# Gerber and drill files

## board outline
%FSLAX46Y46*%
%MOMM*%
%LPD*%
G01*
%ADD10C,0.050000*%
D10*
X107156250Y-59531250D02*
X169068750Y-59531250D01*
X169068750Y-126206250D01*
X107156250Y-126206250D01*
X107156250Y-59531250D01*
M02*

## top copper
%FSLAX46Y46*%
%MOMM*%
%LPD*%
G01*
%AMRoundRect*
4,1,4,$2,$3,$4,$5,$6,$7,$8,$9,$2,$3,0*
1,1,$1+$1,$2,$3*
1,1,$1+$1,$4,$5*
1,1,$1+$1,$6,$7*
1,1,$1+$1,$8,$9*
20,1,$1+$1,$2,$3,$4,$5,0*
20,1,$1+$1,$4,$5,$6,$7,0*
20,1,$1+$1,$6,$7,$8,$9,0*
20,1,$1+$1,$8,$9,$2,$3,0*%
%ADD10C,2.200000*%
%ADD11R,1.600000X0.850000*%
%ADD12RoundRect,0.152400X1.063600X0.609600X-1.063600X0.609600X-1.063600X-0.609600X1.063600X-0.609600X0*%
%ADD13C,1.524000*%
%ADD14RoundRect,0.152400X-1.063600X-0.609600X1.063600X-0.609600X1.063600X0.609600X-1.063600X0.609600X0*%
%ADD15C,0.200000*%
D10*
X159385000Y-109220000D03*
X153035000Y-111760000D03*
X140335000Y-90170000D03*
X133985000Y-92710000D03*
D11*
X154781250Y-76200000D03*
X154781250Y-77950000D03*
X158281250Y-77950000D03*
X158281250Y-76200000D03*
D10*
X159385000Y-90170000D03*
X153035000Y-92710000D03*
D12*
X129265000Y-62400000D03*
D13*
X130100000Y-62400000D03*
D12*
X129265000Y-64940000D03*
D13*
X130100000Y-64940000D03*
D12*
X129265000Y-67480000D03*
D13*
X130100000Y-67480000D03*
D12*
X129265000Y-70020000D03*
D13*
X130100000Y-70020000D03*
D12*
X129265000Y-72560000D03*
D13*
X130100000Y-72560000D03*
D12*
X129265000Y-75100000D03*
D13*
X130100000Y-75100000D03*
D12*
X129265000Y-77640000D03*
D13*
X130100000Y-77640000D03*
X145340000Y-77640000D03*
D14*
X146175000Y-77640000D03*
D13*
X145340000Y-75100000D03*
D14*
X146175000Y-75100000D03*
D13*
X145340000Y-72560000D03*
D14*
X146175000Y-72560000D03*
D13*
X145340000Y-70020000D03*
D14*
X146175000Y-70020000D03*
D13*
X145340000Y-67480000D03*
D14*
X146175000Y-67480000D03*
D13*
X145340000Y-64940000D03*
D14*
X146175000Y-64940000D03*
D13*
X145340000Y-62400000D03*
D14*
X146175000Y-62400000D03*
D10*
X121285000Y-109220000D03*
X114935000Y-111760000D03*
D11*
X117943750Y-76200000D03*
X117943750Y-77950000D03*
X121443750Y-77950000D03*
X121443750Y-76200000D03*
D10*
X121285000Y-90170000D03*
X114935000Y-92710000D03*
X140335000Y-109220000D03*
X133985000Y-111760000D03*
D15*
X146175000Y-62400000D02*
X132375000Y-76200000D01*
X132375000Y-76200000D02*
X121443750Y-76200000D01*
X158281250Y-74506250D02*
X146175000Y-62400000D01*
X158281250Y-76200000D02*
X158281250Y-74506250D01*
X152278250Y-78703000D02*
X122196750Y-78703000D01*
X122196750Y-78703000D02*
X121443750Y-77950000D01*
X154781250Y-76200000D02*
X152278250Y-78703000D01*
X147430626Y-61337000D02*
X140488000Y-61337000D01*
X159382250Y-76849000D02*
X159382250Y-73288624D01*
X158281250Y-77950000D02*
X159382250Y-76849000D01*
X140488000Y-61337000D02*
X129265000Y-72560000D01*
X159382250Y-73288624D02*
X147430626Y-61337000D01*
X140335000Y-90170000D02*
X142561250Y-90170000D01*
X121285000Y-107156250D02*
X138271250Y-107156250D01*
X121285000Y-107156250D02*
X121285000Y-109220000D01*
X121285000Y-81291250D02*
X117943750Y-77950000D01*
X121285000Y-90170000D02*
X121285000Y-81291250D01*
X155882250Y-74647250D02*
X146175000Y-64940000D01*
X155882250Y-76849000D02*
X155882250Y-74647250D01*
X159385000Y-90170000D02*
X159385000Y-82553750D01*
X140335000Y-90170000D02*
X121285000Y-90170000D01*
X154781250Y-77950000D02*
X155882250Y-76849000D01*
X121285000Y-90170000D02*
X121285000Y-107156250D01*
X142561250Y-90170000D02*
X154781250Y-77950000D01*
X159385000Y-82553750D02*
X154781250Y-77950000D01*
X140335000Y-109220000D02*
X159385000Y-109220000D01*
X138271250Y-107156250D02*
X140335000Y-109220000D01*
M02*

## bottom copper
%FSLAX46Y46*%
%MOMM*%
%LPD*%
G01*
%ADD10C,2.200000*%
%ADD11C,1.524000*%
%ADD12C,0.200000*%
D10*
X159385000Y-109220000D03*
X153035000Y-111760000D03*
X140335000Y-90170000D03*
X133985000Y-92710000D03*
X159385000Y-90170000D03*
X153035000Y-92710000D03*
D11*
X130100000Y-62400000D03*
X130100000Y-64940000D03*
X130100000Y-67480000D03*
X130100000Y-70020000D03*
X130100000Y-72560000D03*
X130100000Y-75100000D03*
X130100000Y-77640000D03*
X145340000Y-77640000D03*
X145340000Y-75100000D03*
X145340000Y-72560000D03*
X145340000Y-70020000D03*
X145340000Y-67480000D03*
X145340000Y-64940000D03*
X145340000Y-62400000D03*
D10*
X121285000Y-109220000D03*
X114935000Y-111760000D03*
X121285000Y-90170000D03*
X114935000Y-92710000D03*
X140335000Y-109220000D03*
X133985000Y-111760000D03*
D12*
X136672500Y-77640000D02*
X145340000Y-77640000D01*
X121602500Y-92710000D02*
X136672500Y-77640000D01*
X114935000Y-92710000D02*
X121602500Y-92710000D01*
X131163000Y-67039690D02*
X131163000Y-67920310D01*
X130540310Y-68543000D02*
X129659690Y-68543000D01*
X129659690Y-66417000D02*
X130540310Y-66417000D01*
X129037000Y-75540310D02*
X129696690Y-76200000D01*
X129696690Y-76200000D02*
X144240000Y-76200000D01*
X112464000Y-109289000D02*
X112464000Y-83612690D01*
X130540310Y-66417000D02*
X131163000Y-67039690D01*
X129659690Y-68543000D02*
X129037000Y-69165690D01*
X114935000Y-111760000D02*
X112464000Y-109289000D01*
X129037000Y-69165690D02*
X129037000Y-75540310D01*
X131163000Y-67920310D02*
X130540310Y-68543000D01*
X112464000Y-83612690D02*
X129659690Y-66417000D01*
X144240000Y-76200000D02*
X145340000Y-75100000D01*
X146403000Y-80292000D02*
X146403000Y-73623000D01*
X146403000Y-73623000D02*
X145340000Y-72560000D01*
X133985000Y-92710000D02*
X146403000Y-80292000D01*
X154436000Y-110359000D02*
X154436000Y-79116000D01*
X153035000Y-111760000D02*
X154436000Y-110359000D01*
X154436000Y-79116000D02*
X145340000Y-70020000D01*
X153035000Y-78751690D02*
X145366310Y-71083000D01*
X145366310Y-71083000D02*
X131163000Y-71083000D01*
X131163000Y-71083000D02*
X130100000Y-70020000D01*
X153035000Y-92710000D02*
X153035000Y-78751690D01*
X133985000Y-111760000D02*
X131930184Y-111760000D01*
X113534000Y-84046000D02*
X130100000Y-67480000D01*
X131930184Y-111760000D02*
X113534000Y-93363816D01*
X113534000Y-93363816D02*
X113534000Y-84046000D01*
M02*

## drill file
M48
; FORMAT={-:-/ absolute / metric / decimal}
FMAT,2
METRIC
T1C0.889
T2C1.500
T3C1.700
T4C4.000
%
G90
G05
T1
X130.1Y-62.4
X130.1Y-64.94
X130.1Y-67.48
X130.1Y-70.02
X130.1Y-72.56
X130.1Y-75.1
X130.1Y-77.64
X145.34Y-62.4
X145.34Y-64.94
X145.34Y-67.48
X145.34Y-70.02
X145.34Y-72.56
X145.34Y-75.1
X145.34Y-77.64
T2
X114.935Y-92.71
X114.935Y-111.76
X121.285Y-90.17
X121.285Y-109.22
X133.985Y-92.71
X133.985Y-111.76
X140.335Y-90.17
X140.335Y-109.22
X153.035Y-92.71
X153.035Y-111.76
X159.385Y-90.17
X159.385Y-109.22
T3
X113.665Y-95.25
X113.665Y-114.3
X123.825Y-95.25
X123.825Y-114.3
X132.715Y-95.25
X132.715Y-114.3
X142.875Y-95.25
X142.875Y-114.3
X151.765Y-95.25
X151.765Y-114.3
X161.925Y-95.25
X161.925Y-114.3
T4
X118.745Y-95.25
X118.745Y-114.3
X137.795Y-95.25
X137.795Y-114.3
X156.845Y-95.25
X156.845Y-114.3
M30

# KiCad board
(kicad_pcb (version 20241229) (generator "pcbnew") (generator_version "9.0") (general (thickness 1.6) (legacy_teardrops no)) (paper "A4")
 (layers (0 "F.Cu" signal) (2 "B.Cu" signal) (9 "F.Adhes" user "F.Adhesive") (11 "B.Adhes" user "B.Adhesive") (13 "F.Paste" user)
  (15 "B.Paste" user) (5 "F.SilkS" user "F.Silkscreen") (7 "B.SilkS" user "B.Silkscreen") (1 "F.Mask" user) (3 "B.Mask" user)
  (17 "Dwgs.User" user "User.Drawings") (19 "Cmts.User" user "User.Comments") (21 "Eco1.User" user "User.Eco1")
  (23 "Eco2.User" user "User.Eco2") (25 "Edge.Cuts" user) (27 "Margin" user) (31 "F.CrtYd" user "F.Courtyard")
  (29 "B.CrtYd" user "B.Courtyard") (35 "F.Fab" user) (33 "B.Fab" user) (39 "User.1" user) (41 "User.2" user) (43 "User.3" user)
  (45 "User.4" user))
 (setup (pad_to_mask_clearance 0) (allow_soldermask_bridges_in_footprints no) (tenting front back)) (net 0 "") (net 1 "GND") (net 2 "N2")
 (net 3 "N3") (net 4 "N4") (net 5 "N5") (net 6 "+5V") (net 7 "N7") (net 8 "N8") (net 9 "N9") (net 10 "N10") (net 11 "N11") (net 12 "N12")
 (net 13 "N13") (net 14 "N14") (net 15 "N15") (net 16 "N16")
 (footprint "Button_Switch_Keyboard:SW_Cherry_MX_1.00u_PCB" (layer "F.Cu") (at 159.385 109.22)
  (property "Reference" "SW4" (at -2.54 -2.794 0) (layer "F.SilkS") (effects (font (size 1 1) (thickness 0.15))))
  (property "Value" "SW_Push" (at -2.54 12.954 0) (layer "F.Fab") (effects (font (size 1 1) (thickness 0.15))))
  (pad "" np_thru_hole circle (at -7.62 5.08) (size 1.7 1.7) (drill 1.7) (layers "*.Cu" "*.Mask"))
  (pad "" np_thru_hole circle (at -2.54 5.08) (size 4 4) (drill 4) (layers "*.Cu" "*.Mask"))
  (pad "" np_thru_hole circle (at 2.54 5.08) (size 1.7 1.7) (drill 1.7) (layers "*.Cu" "*.Mask"))
  (pad "1" thru_hole circle (at 0 0) (size 2.2 2.2) (drill 1.5) (layers "*.Cu" "*.Mask") (remove_unused_layers no) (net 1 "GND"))
  (pad "2" thru_hole circle (at -6.35 2.54) (size 2.2 2.2) (drill 1.5) (layers "*.Cu" "*.Mask") (remove_unused_layers no) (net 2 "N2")))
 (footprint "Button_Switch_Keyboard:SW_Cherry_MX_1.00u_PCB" (layer "F.Cu") (at 140.335 90.17)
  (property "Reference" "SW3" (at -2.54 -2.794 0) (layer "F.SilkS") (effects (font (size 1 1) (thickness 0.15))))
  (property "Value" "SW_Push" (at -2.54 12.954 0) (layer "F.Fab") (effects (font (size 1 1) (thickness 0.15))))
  (pad "" np_thru_hole circle (at -7.62 5.08) (size 1.7 1.7) (drill 1.7) (layers "*.Cu" "*.Mask"))
  (pad "" np_thru_hole circle (at -2.54 5.08) (size 4 4) (drill 4) (layers "*.Cu" "*.Mask"))
  (pad "" np_thru_hole circle (at 2.54 5.08) (size 1.7 1.7) (drill 1.7) (layers "*.Cu" "*.Mask"))
  (pad "1" thru_hole circle (at 0 0) (size 2.2 2.2) (drill 1.5) (layers "*.Cu" "*.Mask") (remove_unused_layers no) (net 1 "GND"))
  (pad "2" thru_hole circle (at -6.35 2.54) (size 2.2 2.2) (drill 1.5) (layers "*.Cu" "*.Mask") (remove_unused_layers no) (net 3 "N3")))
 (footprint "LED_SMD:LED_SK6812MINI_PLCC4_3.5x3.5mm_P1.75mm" (layer "F.Cu") (at 156.53125 77.075)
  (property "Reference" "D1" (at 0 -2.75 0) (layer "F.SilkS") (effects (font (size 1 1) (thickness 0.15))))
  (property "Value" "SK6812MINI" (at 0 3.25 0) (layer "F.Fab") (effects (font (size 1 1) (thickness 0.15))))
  (pad "1" smd rect (at -1.75 -0.875) (size 1.6 0.85) (layers "F.Cu" "F.Mask" "F.Paste") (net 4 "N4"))
  (pad "2" smd rect (at -1.75 0.875) (size 1.6 0.85) (layers "F.Cu" "F.Mask" "F.Paste") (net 1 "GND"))
  (pad "3" smd rect (at 1.75 0.875) (size 1.6 0.85) (layers "F.Cu" "F.Mask" "F.Paste") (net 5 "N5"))
  (pad "4" smd rect (at 1.75 -0.875) (size 1.6 0.85) (layers "F.Cu" "F.Mask" "F.Paste") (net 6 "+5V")))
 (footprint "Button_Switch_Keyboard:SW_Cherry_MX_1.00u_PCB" (layer "F.Cu") (at 159.385 90.17)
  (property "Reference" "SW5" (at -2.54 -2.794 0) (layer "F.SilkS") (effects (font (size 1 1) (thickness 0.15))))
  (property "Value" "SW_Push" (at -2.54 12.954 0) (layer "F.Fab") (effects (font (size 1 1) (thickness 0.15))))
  (pad "" np_thru_hole circle (at -7.62 5.08) (size 1.7 1.7) (drill 1.7) (layers "*.Cu" "*.Mask"))
  (pad "" np_thru_hole circle (at -2.54 5.08) (size 4 4) (drill 4) (layers "*.Cu" "*.Mask"))
  (pad "" np_thru_hole circle (at 2.54 5.08) (size 1.7 1.7) (drill 1.7) (layers "*.Cu" "*.Mask"))
  (pad "1" thru_hole circle (at 0 0) (size 2.2 2.2) (drill 1.5) (layers "*.Cu" "*.Mask") (remove_unused_layers no) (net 1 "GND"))
  (pad "2" thru_hole circle (at -6.35 2.54) (size 2.2 2.2) (drill 1.5) (layers "*.Cu" "*.Mask") (remove_unused_layers no) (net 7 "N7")))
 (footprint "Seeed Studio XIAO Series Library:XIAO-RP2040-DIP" (layer "F.Cu") (at 137.72 70.02)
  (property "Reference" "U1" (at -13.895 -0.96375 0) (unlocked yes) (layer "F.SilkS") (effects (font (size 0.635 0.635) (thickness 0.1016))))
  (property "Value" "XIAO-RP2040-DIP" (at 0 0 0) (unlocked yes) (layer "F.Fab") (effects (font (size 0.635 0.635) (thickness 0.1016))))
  (pad "1" smd roundrect (at -8.455 -7.62 180) (size 2.432 1.524) (layers "F.Cu" "F.Mask") (roundrect_rratio 0.1) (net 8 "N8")
   (thermal_bridge_angle 45))
  (pad "1" thru_hole circle (at -7.62 -7.62 180) (size 1.524 1.524) (drill 0.889) (layers "*.Cu" "*.Mask") (remove_unused_layers no)
   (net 8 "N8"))
  (pad "2" smd roundrect (at -8.455 -5.08 180) (size 2.432 1.524) (layers "F.Cu" "F.Mask") (roundrect_rratio 0.1) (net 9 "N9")
   (thermal_bridge_angle 45))
  (pad "2" thru_hole circle (at -7.62 -5.08 180) (size 1.524 1.524) (drill 0.889) (layers "*.Cu" "*.Mask") (remove_unused_layers no)
   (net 9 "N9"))
  (pad "3" smd roundrect (at -8.455 -2.54 180) (size 2.432 1.524) (layers "F.Cu" "F.Mask") (roundrect_rratio 0.1) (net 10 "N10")
   (thermal_bridge_angle 45))
  (pad "3" thru_hole circle (at -7.62 -2.54 180) (size 1.524 1.524) (drill 0.889) (layers "*.Cu" "*.Mask") (remove_unused_layers no)
   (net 10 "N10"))
  (pad "4" smd roundrect (at -8.455 0 180) (size 2.432 1.524) (layers "F.Cu" "F.Mask") (roundrect_rratio 0.1) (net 7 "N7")
   (thermal_bridge_angle 45))
  (pad "4" thru_hole circle (at -7.62 0 180) (size 1.524 1.524) (drill 0.889) (layers "*.Cu" "*.Mask") (remove_unused_layers no)
   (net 7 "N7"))
  (pad "5" smd roundrect (at -8.455 2.54 180) (size 2.432 1.524) (layers "F.Cu" "F.Mask") (roundrect_rratio 0.1) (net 5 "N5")
   (thermal_bridge_angle 45))
  (pad "5" thru_hole circle (at -7.62 2.54 180) (size 1.524 1.524) (drill 0.889) (layers "*.Cu" "*.Mask") (remove_unused_layers no)
   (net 5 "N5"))
  (pad "6" smd roundrect (at -8.455 5.08 180) (size 2.432 1.524) (layers "F.Cu" "F.Mask") (roundrect_rratio 0.1) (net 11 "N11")
   (thermal_bridge_angle 45))
  (pad "6" thru_hole circle (at -7.62 5.08 180) (size 1.524 1.524) (drill 0.889) (layers "*.Cu" "*.Mask") (remove_unused_layers no)
   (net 11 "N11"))
  (pad "7" smd roundrect (at -8.455 7.62 180) (size 2.432 1.524) (layers "F.Cu" "F.Mask") (roundrect_rratio 0.1) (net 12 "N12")
   (thermal_bridge_angle 45))
  (pad "7" thru_hole circle (at -7.62 7.62 180) (size 1.524 1.524) (drill 0.889) (layers "*.Cu" "*.Mask") (remove_unused_layers no)
   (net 12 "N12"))
  (pad "8" thru_hole circle (at 7.62 7.62) (size 1.524 1.524) (drill 0.889) (layers "*.Cu" "*.Mask") (remove_unused_layers no)
   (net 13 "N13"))
  (pad "8" smd roundrect (at 8.455 7.62) (size 2.432 1.524) (layers "F.Cu" "F.Mask") (roundrect_rratio 0.1) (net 13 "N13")
   (thermal_bridge_angle 45))
  (pad "9" thru_hole circle (at 7.62 5.08) (size 1.524 1.524) (drill 0.889) (layers "*.Cu" "*.Mask") (remove_unused_layers no)
   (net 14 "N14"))
  (pad "9" smd roundrect (at 8.455 5.08) (size 2.432 1.524) (layers "F.Cu" "F.Mask") (roundrect_rratio 0.1) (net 14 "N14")
   (thermal_bridge_angle 45))
  (pad "10" thru_hole circle (at 7.62 2.54) (size 1.524 1.524) (drill 0.889) (layers "*.Cu" "*.Mask") (remove_unused_layers no) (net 3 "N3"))
  (pad "10" smd roundrect (at 8.455 2.54) (size 2.432 1.524) (layers "F.Cu" "F.Mask") (roundrect_rratio 0.1) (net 3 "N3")
   (thermal_bridge_angle 45))
  (pad "11" thru_hole circle (at 7.62 0) (size 1.524 1.524) (drill 0.889) (layers "*.Cu" "*.Mask") (remove_unused_layers no) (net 2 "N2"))
  (pad "11" smd roundrect (at 8.455 0) (size 2.432 1.524) (layers "F.Cu" "F.Mask") (roundrect_rratio 0.1) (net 2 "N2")
   (thermal_bridge_angle 45))
  (pad "12" thru_hole circle (at 7.62 -2.54) (size 1.524 1.524) (drill 0.889) (layers "*.Cu" "*.Mask") (remove_unused_layers no)
   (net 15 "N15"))
  (pad "12" smd roundrect (at 8.455 -2.54) (size 2.432 1.524) (layers "F.Cu" "F.Mask") (roundrect_rratio 0.1) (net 15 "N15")
   (thermal_bridge_angle 45))
  (pad "13" thru_hole circle (at 7.62 -5.08) (size 1.524 1.524) (drill 0.889) (layers "*.Cu" "*.Mask") (remove_unused_layers no)
   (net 1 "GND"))
  (pad "13" smd roundrect (at 8.455 -5.08) (size 2.432 1.524) (layers "F.Cu" "F.Mask") (roundrect_rratio 0.1) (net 1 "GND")
   (thermal_bridge_angle 45))
  (pad "14" thru_hole circle (at 7.62 -7.62) (size 1.524 1.524) (drill 0.889) (layers "*.Cu" "*.Mask") (remove_unused_layers no)
   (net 6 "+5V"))
  (pad "14" smd roundrect (at 8.455 -7.62) (size 2.432 1.524) (layers "F.Cu" "F.Mask") (roundrect_rratio 0.1) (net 6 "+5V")
   (thermal_bridge_angle 45)))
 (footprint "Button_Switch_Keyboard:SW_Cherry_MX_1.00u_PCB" (layer "F.Cu") (at 121.285 109.22)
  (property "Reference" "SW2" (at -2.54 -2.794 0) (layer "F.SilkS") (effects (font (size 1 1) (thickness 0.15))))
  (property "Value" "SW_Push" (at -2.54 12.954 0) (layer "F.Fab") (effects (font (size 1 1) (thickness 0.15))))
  (pad "" np_thru_hole circle (at -7.62 5.08) (size 1.7 1.7) (drill 1.7) (layers "*.Cu" "*.Mask"))
  (pad "" np_thru_hole circle (at -2.54 5.08) (size 4 4) (drill 4) (layers "*.Cu" "*.Mask"))
  (pad "" np_thru_hole circle (at 2.54 5.08) (size 1.7 1.7) (drill 1.7) (layers "*.Cu" "*.Mask"))
  (pad "1" thru_hole circle (at 0 0) (size 2.2 2.2) (drill 1.5) (layers "*.Cu" "*.Mask") (remove_unused_layers no) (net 1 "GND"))
  (pad "2" thru_hole circle (at -6.35 2.54) (size 2.2 2.2) (drill 1.5) (layers "*.Cu" "*.Mask") (remove_unused_layers no) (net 14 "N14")))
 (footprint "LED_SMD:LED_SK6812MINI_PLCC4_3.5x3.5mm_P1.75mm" (layer "F.Cu") (at 119.69375 77.075)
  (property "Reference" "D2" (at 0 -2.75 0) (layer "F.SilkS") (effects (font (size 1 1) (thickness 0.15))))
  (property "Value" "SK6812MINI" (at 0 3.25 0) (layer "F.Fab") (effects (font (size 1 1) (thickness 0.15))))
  (pad "1" smd rect (at -1.75 -0.875) (size 1.6 0.85) (layers "F.Cu" "F.Mask" "F.Paste") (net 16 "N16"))
  (pad "2" smd rect (at -1.75 0.875) (size 1.6 0.85) (layers "F.Cu" "F.Mask" "F.Paste") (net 1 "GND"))
  (pad "3" smd rect (at 1.75 0.875) (size 1.6 0.85) (layers "F.Cu" "F.Mask" "F.Paste") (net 4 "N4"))
  (pad "4" smd rect (at 1.75 -0.875) (size 1.6 0.85) (layers "F.Cu" "F.Mask" "F.Paste") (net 6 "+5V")))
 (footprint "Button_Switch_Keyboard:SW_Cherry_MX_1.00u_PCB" (layer "F.Cu") (at 121.285 90.17)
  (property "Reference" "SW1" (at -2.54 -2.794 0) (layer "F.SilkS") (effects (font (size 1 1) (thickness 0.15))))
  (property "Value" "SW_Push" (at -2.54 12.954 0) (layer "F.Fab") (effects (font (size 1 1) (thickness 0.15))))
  (pad "" np_thru_hole circle (at -7.62 5.08) (size 1.7 1.7) (drill 1.7) (layers "*.Cu" "*.Mask"))
  (pad "" np_thru_hole circle (at -2.54 5.08) (size 4 4) (drill 4) (layers "*.Cu" "*.Mask"))
  (pad "" np_thru_hole circle (at 2.54 5.08) (size 1.7 1.7) (drill 1.7) (layers "*.Cu" "*.Mask"))
  (pad "1" thru_hole circle (at 0 0) (size 2.2 2.2) (drill 1.5) (layers "*.Cu" "*.Mask") (remove_unused_layers no) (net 1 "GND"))
  (pad "2" thru_hole circle (at -6.35 2.54) (size 2.2 2.2) (drill 1.5) (layers "*.Cu" "*.Mask") (remove_unused_layers no) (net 13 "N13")))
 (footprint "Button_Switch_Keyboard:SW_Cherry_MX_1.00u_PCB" (layer "F.Cu") (at 140.335 109.22)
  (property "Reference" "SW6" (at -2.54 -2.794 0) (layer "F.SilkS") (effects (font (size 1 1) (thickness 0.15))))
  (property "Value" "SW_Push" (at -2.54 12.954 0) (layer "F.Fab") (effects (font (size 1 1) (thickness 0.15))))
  (pad "" np_thru_hole circle (at -7.62 5.08) (size 1.7 1.7) (drill 1.7) (layers "*.Cu" "*.Mask"))
  (pad "" np_thru_hole circle (at -2.54 5.08) (size 4 4) (drill 4) (layers "*.Cu" "*.Mask"))
  (pad "" np_thru_hole circle (at 2.54 5.08) (size 1.7 1.7) (drill 1.7) (layers "*.Cu" "*.Mask"))
  (pad "1" thru_hole circle (at 0 0) (size 2.2 2.2) (drill 1.5) (layers "*.Cu" "*.Mask") (remove_unused_layers no) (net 1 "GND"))
  (pad "2" thru_hole circle (at -6.35 2.54) (size 2.2 2.2) (drill 1.5) (layers "*.Cu" "*.Mask") (remove_unused_layers no) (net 10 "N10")))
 (gr_rect (start 107.15625 59.53125) (end 169.06875 126.20625) (stroke (width 0.05) (type default)) (fill no) (layer "Edge.Cuts"))
 (segment (start 146.175 62.4) (end 132.375 76.2) (width 0.2) (layer "F.Cu") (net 6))
 (segment (start 132.375 76.2) (end 121.44375 76.2) (width 0.2) (layer "F.Cu") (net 6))
 (segment (start 158.28125 74.50625) (end 146.175 62.4) (width 0.2) (layer "F.Cu") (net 6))
 (segment (start 158.28125 76.2) (end 158.28125 74.50625) (width 0.2) (layer "F.Cu") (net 6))
 (segment (start 152.27825 78.703) (end 122.19675 78.703) (width 0.2) (layer "F.Cu") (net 4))
 (segment (start 122.19675 78.703) (end 121.44375 77.95) (width 0.2) (layer "F.Cu") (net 4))
 (segment (start 154.78125 76.2) (end 152.27825 78.703) (width 0.2) (layer "F.Cu") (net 4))
 (segment (start 147.430626 61.337) (end 140.488 61.337) (width 0.2) (layer "F.Cu") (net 5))
 (segment (start 159.38225 76.849) (end 159.38225 73.288624) (width 0.2) (layer "F.Cu") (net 5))
 (segment (start 158.28125 77.95) (end 159.38225 76.849) (width 0.2) (layer "F.Cu") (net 5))
 (segment (start 140.488 61.337) (end 129.265 72.56) (width 0.2) (layer "F.Cu") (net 5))
 (segment (start 159.38225 73.288624) (end 147.430626 61.337) (width 0.2) (layer "F.Cu") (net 5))
 (segment (start 140.335 90.17) (end 142.56125 90.17) (width 0.2) (layer "F.Cu") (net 1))
 (segment (start 121.285 107.15625) (end 138.27125 107.15625) (width 0.2) (layer "F.Cu") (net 1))
 (segment (start 121.285 107.15625) (end 121.285 109.22) (width 0.2) (layer "F.Cu") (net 1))
 (segment (start 121.285 81.29125) (end 117.94375 77.95) (width 0.2) (layer "F.Cu") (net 1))
 (segment (start 121.285 90.17) (end 121.285 81.29125) (width 0.2) (layer "F.Cu") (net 1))
 (segment (start 155.88225 74.64725) (end 146.175 64.94) (width 0.2) (layer "F.Cu") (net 1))
 (segment (start 155.88225 76.849) (end 155.88225 74.64725) (width 0.2) (layer "F.Cu") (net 1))
 (segment (start 159.385 90.17) (end 159.385 82.55375) (width 0.2) (layer "F.Cu") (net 1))
 (segment (start 140.335 90.17) (end 121.285 90.17) (width 0.2) (layer "F.Cu") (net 1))
 (segment (start 154.78125 77.95) (end 155.88225 76.849) (width 0.2) (layer "F.Cu") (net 1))
 (segment (start 121.285 90.17) (end 121.285 107.15625) (width 0.2) (layer "F.Cu") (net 1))
 (segment (start 142.56125 90.17) (end 154.78125 77.95) (width 0.2) (layer "F.Cu") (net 1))
 (segment (start 159.385 82.55375) (end 154.78125 77.95) (width 0.2) (layer "F.Cu") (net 1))
 (segment (start 140.335 109.22) (end 159.385 109.22) (width 0.2) (layer "F.Cu") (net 1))
 (segment (start 138.27125 107.15625) (end 140.335 109.22) (width 0.2) (layer "F.Cu") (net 1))
 (segment (start 136.6725 77.64) (end 145.34 77.64) (width 0.2) (layer "B.Cu") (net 13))
 (segment (start 121.6025 92.71) (end 136.6725 77.64) (width 0.2) (layer "B.Cu") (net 13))
 (segment (start 114.935 92.71) (end 121.6025 92.71) (width 0.2) (layer "B.Cu") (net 13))
 (segment (start 131.163 67.03969) (end 131.163 67.92031) (width 0.2) (layer "B.Cu") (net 14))
 (segment (start 130.54031 68.543) (end 129.65969 68.543) (width 0.2) (layer "B.Cu") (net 14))
 (segment (start 129.65969 66.417) (end 130.54031 66.417) (width 0.2) (layer "B.Cu") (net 14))
 (segment (start 129.037 75.54031) (end 129.69669 76.2) (width 0.2) (layer "B.Cu") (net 14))
 (segment (start 129.69669 76.2) (end 144.24 76.2) (width 0.2) (layer "B.Cu") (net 14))
 (segment (start 112.464 109.289) (end 112.464 83.61269) (width 0.2) (layer "B.Cu") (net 14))
 (segment (start 130.54031 66.417) (end 131.163 67.03969) (width 0.2) (layer "B.Cu") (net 14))
 (segment (start 129.65969 68.543) (end 129.037 69.16569) (width 0.2) (layer "B.Cu") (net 14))
 (segment (start 114.935 111.76) (end 112.464 109.289) (width 0.2) (layer "B.Cu") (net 14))
 (segment (start 129.037 69.16569) (end 129.037 75.54031) (width 0.2) (layer "B.Cu") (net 14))
 (segment (start 131.163 67.92031) (end 130.54031 68.543) (width 0.2) (layer "B.Cu") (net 14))
 (segment (start 112.464 83.61269) (end 129.65969 66.417) (width 0.2) (layer "B.Cu") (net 14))
 (segment (start 144.24 76.2) (end 145.34 75.1) (width 0.2) (layer "B.Cu") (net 14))
 (segment (start 146.403 80.292) (end 146.403 73.623) (width 0.2) (layer "B.Cu") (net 3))
 (segment (start 146.403 73.623) (end 145.34 72.56) (width 0.2) (layer "B.Cu") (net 3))
 (segment (start 133.985 92.71) (end 146.403 80.292) (width 0.2) (layer "B.Cu") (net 3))
 (segment (start 154.436 110.359) (end 154.436 79.116) (width 0.2) (layer "B.Cu") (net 2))
 (segment (start 153.035 111.76) (end 154.436 110.359) (width 0.2) (layer "B.Cu") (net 2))
 (segment (start 154.436 79.116) (end 145.34 70.02) (width 0.2) (layer "B.Cu") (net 2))
 (segment (start 153.035 78.75169) (end 145.36631 71.083) (width 0.2) (layer "B.Cu") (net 7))
 (segment (start 145.36631 71.083) (end 131.163 71.083) (width 0.2) (layer "B.Cu") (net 7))
 (segment (start 131.163 71.083) (end 130.1 70.02) (width 0.2) (layer "B.Cu") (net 7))
 (segment (start 153.035 92.71) (end 153.035 78.75169) (width 0.2) (layer "B.Cu") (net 7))
 (segment (start 133.985 111.76) (end 131.930184 111.76) (width 0.2) (layer "B.Cu") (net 10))
 (segment (start 113.534 84.046) (end 130.1 67.48) (width 0.2) (layer "B.Cu") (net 10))
 (segment (start 131.930184 111.76) (end 113.534 93.363816) (width 0.2) (layer "B.Cu") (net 10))
 (segment (start 113.534 93.363816) (end 113.534 84.046) (width 0.2) (layer "B.Cu") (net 10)))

